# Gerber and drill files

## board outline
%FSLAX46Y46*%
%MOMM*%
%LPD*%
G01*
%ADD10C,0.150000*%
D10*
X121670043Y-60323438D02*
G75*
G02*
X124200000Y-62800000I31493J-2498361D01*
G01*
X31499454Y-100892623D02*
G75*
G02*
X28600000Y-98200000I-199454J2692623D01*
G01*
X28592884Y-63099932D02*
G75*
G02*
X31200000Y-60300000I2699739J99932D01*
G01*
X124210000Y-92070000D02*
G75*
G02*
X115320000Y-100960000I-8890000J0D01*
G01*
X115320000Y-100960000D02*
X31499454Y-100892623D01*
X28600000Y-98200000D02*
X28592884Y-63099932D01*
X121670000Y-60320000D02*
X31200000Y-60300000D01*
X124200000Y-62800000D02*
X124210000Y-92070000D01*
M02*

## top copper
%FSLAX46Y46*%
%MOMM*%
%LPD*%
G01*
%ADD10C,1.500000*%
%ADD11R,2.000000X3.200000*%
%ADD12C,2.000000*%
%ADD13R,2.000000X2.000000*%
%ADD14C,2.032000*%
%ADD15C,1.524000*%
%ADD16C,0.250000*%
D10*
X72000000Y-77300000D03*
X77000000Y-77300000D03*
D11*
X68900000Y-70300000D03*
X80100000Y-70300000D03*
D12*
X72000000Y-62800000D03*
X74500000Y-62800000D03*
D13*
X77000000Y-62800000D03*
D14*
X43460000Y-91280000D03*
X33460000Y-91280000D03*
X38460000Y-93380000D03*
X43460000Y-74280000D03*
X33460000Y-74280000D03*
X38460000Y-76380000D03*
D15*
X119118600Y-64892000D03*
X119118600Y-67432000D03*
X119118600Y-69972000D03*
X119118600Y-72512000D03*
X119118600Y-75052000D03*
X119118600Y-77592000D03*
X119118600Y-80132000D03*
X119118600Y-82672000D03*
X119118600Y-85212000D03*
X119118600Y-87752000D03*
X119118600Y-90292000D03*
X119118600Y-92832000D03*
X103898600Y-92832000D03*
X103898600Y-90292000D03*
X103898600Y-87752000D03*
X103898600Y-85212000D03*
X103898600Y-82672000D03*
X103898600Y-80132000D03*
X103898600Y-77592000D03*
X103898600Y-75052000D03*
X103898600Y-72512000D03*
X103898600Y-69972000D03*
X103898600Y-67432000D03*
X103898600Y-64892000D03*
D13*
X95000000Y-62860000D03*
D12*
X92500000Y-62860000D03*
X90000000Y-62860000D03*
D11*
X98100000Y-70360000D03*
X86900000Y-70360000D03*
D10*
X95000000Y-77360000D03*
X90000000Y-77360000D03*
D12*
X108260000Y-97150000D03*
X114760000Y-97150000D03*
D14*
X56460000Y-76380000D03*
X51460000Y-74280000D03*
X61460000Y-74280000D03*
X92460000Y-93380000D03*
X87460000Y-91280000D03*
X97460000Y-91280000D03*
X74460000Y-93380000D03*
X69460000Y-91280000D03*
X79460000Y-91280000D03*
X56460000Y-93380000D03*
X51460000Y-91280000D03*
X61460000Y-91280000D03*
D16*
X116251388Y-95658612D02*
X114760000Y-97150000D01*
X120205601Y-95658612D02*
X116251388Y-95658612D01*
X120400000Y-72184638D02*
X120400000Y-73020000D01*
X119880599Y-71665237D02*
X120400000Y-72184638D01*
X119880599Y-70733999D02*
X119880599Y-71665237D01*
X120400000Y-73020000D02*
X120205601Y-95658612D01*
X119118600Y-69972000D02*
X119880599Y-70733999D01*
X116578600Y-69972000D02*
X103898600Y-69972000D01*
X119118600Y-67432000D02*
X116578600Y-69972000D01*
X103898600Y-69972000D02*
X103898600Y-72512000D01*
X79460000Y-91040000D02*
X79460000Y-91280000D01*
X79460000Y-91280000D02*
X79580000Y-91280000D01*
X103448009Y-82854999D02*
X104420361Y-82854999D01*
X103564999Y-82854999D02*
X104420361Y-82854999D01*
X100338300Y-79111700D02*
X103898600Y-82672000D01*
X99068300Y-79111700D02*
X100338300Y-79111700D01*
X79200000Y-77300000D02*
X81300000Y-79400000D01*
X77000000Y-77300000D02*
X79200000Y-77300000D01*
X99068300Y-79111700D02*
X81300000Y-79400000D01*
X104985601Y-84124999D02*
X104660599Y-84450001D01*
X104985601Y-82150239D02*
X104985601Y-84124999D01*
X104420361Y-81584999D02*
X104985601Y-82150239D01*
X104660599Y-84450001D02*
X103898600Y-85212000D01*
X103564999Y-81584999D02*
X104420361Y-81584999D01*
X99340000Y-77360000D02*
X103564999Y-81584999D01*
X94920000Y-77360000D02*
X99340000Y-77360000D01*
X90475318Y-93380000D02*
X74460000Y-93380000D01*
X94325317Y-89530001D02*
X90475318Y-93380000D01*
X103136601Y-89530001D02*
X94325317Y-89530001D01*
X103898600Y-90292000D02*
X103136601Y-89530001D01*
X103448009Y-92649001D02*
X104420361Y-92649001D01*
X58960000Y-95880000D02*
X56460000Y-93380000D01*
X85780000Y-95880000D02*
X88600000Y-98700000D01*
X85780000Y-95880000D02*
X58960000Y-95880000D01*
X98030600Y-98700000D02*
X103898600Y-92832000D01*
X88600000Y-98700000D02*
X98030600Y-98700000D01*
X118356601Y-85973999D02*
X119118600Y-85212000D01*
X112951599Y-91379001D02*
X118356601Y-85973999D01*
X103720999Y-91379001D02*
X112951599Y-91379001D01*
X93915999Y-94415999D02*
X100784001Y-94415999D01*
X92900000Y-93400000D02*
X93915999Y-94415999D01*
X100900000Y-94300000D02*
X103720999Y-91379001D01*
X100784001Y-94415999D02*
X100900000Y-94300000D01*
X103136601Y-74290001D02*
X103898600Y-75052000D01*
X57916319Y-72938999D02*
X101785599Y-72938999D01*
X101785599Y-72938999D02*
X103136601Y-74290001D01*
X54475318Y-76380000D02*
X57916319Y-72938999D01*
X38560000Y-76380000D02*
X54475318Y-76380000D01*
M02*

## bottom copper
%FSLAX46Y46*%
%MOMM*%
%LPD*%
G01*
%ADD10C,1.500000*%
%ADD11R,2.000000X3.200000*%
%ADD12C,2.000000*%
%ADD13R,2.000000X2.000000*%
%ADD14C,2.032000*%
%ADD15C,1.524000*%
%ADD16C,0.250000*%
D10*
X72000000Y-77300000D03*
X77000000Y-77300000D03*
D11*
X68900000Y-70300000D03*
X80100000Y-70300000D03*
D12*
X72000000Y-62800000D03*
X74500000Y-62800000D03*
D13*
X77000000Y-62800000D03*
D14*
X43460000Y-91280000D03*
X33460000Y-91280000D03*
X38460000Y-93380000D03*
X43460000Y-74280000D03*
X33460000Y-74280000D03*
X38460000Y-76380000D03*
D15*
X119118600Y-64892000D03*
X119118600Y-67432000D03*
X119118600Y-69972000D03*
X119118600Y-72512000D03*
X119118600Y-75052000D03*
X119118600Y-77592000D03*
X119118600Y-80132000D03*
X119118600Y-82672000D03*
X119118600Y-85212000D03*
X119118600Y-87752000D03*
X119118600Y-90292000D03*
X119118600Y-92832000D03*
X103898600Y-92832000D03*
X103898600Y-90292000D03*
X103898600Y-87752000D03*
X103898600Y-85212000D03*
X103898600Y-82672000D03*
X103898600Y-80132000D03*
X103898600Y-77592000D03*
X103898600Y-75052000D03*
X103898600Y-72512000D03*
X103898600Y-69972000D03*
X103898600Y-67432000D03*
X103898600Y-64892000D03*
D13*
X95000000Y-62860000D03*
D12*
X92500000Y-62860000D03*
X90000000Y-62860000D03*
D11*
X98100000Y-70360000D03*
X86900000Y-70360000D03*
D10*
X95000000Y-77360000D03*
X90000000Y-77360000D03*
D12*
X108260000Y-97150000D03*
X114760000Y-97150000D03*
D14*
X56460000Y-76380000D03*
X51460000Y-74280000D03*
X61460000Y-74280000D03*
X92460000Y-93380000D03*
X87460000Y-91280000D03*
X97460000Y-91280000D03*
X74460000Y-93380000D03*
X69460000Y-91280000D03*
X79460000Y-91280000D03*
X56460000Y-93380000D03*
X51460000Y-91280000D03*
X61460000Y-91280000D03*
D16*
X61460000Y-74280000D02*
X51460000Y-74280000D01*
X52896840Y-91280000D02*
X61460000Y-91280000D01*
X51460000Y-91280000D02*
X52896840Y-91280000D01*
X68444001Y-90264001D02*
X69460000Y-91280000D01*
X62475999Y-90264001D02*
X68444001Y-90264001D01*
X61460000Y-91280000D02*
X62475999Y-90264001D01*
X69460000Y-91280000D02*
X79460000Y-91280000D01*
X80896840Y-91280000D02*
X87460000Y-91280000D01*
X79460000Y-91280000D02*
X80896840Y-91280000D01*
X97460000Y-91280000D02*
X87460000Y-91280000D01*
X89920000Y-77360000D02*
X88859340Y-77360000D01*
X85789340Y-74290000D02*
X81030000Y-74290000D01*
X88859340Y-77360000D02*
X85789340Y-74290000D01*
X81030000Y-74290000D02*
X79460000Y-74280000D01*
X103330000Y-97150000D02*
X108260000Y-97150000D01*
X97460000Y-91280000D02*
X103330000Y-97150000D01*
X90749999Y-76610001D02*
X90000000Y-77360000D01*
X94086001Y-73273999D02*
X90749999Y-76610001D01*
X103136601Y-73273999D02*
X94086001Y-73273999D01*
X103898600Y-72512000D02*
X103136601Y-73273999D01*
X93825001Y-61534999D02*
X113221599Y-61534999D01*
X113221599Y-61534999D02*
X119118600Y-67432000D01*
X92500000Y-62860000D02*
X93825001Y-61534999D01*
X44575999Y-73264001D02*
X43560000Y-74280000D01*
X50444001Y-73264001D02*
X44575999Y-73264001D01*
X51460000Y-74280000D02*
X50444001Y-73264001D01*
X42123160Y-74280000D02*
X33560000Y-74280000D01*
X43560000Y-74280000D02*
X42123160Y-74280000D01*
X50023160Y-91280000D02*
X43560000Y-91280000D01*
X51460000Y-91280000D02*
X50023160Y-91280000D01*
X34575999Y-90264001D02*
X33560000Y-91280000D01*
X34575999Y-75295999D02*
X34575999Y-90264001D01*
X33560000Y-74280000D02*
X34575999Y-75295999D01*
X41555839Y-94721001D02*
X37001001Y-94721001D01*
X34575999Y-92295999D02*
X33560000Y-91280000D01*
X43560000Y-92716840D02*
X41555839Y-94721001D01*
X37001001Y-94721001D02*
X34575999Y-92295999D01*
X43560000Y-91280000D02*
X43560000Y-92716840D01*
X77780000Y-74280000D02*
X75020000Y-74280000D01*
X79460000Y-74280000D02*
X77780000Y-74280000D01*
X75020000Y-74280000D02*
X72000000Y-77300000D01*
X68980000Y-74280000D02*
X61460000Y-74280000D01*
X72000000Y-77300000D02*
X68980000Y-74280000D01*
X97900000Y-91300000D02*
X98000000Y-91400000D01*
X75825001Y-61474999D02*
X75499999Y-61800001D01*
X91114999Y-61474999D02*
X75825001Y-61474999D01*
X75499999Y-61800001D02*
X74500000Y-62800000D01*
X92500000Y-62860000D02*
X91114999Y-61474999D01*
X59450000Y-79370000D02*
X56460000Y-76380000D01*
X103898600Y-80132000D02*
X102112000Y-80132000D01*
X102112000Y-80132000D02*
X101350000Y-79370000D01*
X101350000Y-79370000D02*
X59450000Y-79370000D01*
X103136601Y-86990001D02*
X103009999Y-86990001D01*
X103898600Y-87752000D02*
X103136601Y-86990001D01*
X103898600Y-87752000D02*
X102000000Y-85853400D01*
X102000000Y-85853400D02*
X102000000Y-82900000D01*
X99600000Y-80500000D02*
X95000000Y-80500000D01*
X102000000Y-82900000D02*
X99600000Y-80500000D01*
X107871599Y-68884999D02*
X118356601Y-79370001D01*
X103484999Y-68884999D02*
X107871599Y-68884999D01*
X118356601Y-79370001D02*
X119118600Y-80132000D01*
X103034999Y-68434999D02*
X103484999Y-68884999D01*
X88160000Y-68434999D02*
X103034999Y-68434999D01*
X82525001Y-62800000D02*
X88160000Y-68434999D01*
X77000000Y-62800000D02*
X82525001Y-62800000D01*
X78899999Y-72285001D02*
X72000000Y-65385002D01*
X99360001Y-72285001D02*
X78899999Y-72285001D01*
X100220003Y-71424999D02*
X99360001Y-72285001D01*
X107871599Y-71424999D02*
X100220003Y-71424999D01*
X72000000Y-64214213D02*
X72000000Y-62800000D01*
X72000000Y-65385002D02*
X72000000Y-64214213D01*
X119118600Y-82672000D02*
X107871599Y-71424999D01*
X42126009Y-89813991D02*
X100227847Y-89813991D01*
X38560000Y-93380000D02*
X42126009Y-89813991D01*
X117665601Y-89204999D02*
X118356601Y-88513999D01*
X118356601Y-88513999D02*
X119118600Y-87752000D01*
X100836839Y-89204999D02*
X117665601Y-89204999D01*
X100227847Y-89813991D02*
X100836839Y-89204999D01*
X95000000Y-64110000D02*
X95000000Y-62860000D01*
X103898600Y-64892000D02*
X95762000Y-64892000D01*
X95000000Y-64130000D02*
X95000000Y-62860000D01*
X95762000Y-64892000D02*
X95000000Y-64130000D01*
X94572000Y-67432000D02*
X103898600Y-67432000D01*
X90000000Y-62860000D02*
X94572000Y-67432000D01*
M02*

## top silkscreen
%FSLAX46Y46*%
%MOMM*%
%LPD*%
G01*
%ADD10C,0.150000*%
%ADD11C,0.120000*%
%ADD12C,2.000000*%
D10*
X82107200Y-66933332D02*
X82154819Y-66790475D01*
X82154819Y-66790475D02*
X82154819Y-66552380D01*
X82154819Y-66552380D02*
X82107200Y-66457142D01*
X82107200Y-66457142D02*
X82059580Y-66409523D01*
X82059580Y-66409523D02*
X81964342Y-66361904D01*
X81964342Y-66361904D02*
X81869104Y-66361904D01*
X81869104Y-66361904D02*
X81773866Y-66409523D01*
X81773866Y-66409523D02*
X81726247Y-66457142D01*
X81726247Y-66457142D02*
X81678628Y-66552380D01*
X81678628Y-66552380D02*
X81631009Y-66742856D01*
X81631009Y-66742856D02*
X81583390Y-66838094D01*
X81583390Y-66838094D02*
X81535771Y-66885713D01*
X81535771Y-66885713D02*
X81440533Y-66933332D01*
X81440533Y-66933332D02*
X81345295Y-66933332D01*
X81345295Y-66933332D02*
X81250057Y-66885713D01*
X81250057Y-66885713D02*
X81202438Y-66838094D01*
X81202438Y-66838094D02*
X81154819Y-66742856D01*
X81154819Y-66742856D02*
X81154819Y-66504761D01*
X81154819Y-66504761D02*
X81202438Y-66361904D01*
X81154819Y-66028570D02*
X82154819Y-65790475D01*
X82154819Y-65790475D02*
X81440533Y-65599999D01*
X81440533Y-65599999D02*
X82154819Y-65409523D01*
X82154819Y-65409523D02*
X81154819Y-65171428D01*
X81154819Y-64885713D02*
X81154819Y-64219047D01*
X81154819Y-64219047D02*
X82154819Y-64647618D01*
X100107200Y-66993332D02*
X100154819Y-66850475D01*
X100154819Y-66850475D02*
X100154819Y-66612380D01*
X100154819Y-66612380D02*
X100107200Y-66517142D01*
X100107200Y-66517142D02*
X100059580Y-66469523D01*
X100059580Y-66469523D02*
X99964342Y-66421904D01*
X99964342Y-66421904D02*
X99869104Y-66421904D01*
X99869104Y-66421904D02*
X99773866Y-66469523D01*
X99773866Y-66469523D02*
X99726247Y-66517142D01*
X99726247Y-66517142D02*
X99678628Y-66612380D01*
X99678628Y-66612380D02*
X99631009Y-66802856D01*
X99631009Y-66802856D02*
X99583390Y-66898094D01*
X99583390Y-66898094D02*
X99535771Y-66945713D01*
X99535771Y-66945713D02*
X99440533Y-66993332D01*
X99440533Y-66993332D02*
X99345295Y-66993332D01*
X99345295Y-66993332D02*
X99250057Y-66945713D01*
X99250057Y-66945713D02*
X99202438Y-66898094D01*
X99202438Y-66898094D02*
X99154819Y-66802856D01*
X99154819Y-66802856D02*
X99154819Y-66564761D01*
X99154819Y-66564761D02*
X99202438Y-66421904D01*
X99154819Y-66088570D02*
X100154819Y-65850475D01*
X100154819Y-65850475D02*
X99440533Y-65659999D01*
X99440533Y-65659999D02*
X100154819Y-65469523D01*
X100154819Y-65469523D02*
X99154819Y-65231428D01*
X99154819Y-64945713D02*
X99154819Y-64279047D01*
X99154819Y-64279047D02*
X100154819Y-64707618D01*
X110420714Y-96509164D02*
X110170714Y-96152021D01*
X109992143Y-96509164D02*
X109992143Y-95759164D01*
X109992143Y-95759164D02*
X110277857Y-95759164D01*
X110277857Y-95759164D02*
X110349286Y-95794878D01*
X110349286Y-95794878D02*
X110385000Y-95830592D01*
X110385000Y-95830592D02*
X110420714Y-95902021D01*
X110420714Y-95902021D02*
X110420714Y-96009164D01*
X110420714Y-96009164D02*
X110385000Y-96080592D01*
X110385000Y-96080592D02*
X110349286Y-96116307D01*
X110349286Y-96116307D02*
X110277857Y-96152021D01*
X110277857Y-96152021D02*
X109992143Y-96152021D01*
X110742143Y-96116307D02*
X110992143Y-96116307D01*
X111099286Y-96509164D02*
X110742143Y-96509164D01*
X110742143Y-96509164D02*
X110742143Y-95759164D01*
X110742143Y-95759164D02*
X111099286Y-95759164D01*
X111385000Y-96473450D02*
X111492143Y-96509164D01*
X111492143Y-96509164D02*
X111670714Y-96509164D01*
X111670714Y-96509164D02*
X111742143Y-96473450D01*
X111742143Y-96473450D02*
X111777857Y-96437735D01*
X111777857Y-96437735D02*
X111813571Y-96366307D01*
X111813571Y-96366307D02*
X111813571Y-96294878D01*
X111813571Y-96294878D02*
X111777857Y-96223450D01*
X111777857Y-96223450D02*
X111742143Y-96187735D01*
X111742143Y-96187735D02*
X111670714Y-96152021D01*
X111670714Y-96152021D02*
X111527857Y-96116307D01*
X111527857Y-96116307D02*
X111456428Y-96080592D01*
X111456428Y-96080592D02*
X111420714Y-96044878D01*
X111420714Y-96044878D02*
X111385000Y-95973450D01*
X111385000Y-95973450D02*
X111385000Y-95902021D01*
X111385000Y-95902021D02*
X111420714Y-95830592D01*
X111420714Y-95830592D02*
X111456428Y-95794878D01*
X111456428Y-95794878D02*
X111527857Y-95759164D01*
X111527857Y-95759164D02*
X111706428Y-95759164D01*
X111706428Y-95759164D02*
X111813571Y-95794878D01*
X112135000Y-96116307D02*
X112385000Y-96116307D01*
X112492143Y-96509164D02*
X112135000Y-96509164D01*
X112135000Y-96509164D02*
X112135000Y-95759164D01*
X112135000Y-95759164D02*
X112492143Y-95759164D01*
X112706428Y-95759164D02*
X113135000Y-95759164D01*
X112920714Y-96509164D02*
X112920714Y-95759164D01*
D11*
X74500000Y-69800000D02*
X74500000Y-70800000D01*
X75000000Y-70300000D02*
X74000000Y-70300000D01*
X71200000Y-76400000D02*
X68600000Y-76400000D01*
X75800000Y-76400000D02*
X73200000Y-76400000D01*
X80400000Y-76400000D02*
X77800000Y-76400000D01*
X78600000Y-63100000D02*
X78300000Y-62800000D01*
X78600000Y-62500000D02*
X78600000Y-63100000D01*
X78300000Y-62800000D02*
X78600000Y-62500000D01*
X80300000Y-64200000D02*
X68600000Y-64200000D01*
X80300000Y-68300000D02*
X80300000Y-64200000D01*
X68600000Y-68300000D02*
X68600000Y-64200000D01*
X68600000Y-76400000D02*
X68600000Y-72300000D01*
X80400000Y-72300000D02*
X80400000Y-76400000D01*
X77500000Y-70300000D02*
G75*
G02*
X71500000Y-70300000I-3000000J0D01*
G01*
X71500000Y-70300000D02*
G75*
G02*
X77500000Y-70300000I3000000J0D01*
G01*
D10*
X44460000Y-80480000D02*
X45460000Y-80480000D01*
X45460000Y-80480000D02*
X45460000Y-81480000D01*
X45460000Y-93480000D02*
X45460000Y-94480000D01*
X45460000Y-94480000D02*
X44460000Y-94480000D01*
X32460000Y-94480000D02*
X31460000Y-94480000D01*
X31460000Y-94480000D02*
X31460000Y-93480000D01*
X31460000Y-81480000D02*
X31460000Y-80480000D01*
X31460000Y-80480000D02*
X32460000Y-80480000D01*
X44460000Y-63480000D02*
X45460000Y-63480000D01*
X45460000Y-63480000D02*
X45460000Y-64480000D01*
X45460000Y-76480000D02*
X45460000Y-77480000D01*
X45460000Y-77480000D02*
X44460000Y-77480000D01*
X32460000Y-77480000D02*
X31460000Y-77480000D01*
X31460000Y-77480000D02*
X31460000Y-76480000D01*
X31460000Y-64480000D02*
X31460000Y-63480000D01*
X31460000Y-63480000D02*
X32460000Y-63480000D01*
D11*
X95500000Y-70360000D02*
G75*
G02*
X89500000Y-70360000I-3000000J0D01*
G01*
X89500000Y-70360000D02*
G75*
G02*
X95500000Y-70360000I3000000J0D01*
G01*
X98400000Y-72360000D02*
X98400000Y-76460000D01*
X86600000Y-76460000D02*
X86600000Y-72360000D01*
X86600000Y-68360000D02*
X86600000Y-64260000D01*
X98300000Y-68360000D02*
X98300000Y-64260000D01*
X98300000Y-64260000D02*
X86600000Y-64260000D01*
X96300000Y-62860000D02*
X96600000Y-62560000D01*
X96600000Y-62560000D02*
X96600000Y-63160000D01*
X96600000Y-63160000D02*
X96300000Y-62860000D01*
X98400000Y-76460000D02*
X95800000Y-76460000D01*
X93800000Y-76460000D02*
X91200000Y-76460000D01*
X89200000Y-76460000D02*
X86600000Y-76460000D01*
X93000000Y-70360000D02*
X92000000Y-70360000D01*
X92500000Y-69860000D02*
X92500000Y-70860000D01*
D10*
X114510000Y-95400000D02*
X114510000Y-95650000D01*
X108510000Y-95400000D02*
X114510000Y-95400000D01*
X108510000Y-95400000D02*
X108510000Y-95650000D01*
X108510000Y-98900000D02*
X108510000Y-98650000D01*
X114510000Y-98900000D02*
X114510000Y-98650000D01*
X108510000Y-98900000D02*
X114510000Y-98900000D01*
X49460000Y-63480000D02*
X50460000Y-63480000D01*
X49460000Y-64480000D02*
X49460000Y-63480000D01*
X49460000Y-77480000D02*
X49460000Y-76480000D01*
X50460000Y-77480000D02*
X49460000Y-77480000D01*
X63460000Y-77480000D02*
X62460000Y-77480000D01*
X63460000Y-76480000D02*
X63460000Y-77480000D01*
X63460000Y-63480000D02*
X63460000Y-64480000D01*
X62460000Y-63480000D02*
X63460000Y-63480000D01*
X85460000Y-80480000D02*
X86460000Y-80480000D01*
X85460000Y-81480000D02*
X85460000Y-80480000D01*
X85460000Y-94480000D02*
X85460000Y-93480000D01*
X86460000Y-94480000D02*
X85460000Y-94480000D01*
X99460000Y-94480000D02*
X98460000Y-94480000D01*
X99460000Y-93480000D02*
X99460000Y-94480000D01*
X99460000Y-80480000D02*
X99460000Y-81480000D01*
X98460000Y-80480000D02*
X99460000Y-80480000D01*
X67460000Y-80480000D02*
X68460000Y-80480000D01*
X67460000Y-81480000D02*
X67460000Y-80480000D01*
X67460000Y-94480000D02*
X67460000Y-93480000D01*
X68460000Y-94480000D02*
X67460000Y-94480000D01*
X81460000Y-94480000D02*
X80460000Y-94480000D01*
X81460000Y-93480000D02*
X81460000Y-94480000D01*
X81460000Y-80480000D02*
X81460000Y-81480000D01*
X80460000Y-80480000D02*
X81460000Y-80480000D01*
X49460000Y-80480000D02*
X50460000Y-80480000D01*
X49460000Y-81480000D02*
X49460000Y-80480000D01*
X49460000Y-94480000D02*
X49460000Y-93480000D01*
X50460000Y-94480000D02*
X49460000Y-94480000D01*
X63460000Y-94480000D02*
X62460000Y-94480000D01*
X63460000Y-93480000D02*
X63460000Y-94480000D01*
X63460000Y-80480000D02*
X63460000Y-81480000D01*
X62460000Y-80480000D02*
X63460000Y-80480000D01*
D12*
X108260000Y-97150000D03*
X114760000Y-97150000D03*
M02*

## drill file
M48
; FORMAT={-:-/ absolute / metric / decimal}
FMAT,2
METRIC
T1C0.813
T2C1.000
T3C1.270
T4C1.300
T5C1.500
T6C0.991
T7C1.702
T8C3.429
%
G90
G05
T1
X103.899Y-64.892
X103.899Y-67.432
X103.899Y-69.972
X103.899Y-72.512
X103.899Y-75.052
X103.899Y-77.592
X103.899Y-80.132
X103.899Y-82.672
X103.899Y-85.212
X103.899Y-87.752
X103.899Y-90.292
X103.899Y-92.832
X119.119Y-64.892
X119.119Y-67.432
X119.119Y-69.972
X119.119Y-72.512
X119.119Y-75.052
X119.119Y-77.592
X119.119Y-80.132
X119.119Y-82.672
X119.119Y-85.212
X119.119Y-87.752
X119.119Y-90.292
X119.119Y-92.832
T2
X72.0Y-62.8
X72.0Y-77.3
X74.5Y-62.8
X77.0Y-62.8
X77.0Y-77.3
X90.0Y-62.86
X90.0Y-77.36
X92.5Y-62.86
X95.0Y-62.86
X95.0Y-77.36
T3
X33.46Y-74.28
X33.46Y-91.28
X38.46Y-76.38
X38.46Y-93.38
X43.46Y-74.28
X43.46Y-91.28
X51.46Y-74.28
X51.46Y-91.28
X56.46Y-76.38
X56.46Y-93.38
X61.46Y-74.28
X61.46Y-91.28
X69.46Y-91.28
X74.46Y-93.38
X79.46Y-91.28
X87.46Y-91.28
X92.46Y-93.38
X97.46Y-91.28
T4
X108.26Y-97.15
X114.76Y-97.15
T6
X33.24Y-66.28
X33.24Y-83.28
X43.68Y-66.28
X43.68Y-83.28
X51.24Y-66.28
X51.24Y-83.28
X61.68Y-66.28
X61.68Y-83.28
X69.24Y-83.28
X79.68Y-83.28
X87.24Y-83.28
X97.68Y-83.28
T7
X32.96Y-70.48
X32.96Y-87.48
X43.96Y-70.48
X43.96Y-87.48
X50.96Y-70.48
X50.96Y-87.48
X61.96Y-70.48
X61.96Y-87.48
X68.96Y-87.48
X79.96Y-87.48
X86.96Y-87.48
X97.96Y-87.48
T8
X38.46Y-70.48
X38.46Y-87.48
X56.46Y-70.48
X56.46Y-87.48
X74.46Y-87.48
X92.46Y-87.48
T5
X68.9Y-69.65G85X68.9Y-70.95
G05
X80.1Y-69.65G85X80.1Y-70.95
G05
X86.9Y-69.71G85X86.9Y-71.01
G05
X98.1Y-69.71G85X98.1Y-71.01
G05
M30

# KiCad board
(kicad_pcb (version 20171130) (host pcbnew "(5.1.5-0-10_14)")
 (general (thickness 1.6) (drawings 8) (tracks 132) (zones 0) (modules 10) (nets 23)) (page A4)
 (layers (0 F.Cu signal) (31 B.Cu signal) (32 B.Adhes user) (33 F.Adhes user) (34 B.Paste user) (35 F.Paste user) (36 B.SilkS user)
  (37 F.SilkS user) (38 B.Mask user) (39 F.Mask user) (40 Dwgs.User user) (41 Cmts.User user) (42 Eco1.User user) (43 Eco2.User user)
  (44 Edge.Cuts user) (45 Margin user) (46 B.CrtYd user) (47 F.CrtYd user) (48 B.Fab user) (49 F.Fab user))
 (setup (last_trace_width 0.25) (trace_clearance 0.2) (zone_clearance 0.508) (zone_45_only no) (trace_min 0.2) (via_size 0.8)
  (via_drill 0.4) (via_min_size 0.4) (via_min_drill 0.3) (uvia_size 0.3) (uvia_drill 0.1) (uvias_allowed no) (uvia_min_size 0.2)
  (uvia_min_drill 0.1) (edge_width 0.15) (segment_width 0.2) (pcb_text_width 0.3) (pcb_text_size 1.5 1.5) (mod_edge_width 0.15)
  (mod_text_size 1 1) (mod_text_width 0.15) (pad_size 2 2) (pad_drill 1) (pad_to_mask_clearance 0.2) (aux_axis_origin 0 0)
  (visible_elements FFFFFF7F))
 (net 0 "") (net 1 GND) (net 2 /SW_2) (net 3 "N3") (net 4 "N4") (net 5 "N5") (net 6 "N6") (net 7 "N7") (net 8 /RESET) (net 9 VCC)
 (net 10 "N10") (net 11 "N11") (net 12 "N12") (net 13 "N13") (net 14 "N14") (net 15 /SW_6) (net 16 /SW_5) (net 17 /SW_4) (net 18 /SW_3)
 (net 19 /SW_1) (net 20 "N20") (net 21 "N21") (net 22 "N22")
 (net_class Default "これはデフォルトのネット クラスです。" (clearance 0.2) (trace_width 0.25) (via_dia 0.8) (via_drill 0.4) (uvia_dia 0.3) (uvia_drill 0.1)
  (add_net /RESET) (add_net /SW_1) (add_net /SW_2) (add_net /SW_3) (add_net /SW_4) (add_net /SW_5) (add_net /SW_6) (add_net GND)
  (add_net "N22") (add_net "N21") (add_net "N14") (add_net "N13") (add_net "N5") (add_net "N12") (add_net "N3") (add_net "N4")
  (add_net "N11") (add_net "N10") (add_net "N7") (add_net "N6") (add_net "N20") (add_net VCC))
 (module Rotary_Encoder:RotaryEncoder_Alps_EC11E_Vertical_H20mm (layer F.Cu) (at 77 62.8 270)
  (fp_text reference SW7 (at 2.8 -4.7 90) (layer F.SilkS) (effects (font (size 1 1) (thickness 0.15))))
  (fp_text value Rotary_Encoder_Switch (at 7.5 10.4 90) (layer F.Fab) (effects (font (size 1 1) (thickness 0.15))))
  (fp_line (start 7 2.5) (end 8 2.5) (layer F.SilkS) (width 0.12))
  (fp_line (start 7.5 2) (end 7.5 3) (layer F.SilkS) (width 0.12))
  (fp_line (start 13.6 5.8) (end 13.6 8.4) (layer F.SilkS) (width 0.12))
  (fp_line (start 13.6 1.2) (end 13.6 3.8) (layer F.SilkS) (width 0.12))
  (fp_line (start 13.6 -3.4) (end 13.6 -0.8) (layer F.SilkS) (width 0.12))
  (fp_line (start 0.3 -1.6) (end 0 -1.3) (layer F.SilkS) (width 0.12))
  (fp_line (start -0.3 -1.6) (end 0.3 -1.6) (layer F.SilkS) (width 0.12))
  (fp_line (start 0 -1.3) (end -0.3 -1.6) (layer F.SilkS) (width 0.12))
  (fp_line (start 1.4 -3.3) (end 1.4 8.4) (layer F.SilkS) (width 0.12))
  (fp_line (start 5.5 -3.3) (end 1.4 -3.3) (layer F.SilkS) (width 0.12))
  (fp_line (start 5.5 8.4) (end 1.4 8.4) (layer F.SilkS) (width 0.12))
  (fp_line (start 13.6 8.4) (end 9.5 8.4) (layer F.SilkS) (width 0.12))
  (fp_line (start 9.5 -3.4) (end 13.6 -3.4) (layer F.SilkS) (width 0.12))
  (fp_circle (center 7.5 2.5) (end 10.5 2.5) (layer F.SilkS) (width 0.12))
  (pad "" thru_hole circle (at 14.5 5 270) (size 1.5 1.5) (drill 1) (layers *.Cu *.Mask) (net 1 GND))
  (pad "" thru_hole circle (at 14.5 0 270) (size 1.5 1.5) (drill 1) (layers *.Cu *.Mask) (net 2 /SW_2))
  (pad MP thru_hole rect (at 7.5 8.1 270) (size 3.2 2) (drill oval 2.8 1.5) (layers *.Cu *.Mask))
  (pad MP thru_hole rect (at 7.5 -3.1 270) (size 3.2 2) (drill oval 2.8 1.5) (layers *.Cu *.Mask))
  (pad B thru_hole circle (at 0 5 270) (size 2 2) (drill 1) (layers *.Cu *.Mask) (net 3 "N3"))
  (pad C thru_hole circle (at 0 2.5 270) (size 2 2) (drill 1) (layers *.Cu *.Mask) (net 1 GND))
  (pad A thru_hole rect (at 0 0 270) (size 2 2) (drill 1) (layers *.Cu *.Mask) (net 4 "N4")))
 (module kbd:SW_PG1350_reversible (layer F.Cu) (at 38.46 87.48)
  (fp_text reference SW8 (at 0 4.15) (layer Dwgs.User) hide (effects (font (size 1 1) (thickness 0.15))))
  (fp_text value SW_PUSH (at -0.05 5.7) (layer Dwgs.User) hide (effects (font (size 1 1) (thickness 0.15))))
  (fp_line (start 6 -7) (end 7 -7) (layer F.SilkS) (width 0.15))
  (fp_line (start 7 -7) (end 7 -6) (layer F.SilkS) (width 0.15)) (fp_line (start 7 6) (end 7 7) (layer F.SilkS) (width 0.15))
  (fp_line (start 7 7) (end 6 7) (layer F.SilkS) (width 0.15))
  (fp_line (start -6 7) (end -7 7) (layer F.SilkS) (width 0.15))
  (fp_line (start -7 7) (end -7 6) (layer F.SilkS) (width 0.15))
  (fp_line (start -7 -6) (end -7 -7) (layer F.SilkS) (width 0.15))
  (fp_line (start -7 -7) (end -6 -7) (layer F.SilkS) (width 0.15))
  (pad "" np_thru_hole circle (at -5.22 -4.2) (size 0.9906 0.9906) (drill 0.9906) (layers *.Cu *.Mask))
  (pad 2 thru_hole circle (at 5 3.8) (size 2.032 2.032) (drill 1.27) (layers *.Cu *.Mask) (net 1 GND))
  (pad "" np_thru_hole circle (at 0 0) (size 3.429 3.429) (drill 3.429) (layers *.Cu *.Mask))
  (pad 2 thru_hole circle (at -5 3.8) (size 2.032 2.032) (drill 1.27) (layers *.Cu *.Mask) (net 1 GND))
  (pad 1 thru_hole circle (at 0 5.9) (size 2.032 2.032) (drill 1.27) (layers *.Cu *.Mask) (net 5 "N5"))
  (pad "" np_thru_hole circle (at 5.22 -4.2) (size 0.9906 0.9906) (drill 0.9906) (layers *.Cu *.Mask))
  (pad "" np_thru_hole circle (at 5.5 0) (size 1.7018 1.7018) (drill 1.7018) (layers *.Cu *.Mask))
  (pad "" np_thru_hole circle (at -5.5 0) (size 1.7018 1.7018) (drill 1.7018) (layers *.Cu *.Mask)))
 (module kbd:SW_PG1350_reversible (layer F.Cu) (at 38.46 70.48)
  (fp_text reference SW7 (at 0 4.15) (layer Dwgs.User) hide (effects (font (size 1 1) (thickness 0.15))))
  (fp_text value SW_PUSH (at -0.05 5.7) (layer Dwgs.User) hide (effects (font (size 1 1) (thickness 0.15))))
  (fp_line (start 6 -7) (end 7 -7) (layer F.SilkS) (width 0.15))
  (fp_line (start 7 -7) (end 7 -6) (layer F.SilkS) (width 0.15)) (fp_line (start 7 6) (end 7 7) (layer F.SilkS) (width 0.15))
  (fp_line (start 7 7) (end 6 7) (layer F.SilkS) (width 0.15))
  (fp_line (start -6 7) (end -7 7) (layer F.SilkS) (width 0.15))
  (fp_line (start -7 7) (end -7 6) (layer F.SilkS) (width 0.15))
  (fp_line (start -7 -6) (end -7 -7) (layer F.SilkS) (width 0.15))
  (fp_line (start -7 -7) (end -6 -7) (layer F.SilkS) (width 0.15))
  (pad "" np_thru_hole circle (at -5.22 -4.2) (size 0.9906 0.9906) (drill 0.9906) (layers *.Cu *.Mask))
  (pad 2 thru_hole circle (at 5 3.8) (size 2.032 2.032) (drill 1.27) (layers *.Cu *.Mask) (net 1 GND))
  (pad "" np_thru_hole circle (at 0 0) (size 3.429 3.429) (drill 3.429) (layers *.Cu *.Mask))
  (pad 2 thru_hole circle (at -5 3.8) (size 2.032 2.032) (drill 1.27) (layers *.Cu *.Mask) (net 1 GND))
  (pad 1 thru_hole circle (at 0 5.9) (size 2.032 2.032) (drill 1.27) (layers *.Cu *.Mask) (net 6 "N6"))
  (pad "" np_thru_hole circle (at 5.22 -4.2) (size 0.9906 0.9906) (drill 0.9906) (layers *.Cu *.Mask))
  (pad "" np_thru_hole circle (at 5.5 0) (size 1.7018 1.7018) (drill 1.7018) (layers *.Cu *.Mask))
  (pad "" np_thru_hole circle (at -5.5 0) (size 1.7018 1.7018) (drill 1.7018) (layers *.Cu *.Mask)))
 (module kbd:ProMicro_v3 (layer B.Cu) (at 111.51 79.37 180)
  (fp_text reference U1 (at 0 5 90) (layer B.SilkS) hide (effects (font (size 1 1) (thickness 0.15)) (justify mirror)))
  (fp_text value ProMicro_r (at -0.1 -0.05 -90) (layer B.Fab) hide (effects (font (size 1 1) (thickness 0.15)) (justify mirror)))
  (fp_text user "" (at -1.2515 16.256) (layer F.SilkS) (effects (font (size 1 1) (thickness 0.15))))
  (pad 24 thru_hole circle (at -7.6086 14.478 180) (size 1.524 1.524) (drill 0.8128) (layers *.Cu *.Mask B.SilkS) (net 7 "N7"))
  (pad 23 thru_hole circle (at -7.6086 11.938 180) (size 1.524 1.524) (drill 0.8128) (layers *.Cu *.Mask B.SilkS) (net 1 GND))
  (pad 22 thru_hole circle (at -7.6086 9.398 180) (size 1.524 1.524) (drill 0.8128) (layers *.Cu *.Mask B.SilkS) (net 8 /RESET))
  (pad 21 thru_hole circle (at -7.6086 6.858 180) (size 1.524 1.524) (drill 0.8128) (layers *.Cu *.Mask B.SilkS) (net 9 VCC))
  (pad 20 thru_hole circle (at -7.6086 4.318 180) (size 1.524 1.524) (drill 0.8128) (layers *.Cu *.Mask B.SilkS) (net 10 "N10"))
  (pad 19 thru_hole circle (at -7.6086 1.778 180) (size 1.524 1.524) (drill 0.8128) (layers *.Cu *.Mask B.SilkS) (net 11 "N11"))
  (pad 18 thru_hole circle (at -7.6086 -0.762 180) (size 1.524 1.524) (drill 0.8128) (layers *.Cu *.Mask B.SilkS) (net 4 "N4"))
  (pad 17 thru_hole circle (at -7.6086 -3.302 180) (size 1.524 1.524) (drill 0.8128) (layers *.Cu *.Mask B.SilkS) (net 3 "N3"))
  (pad 16 thru_hole circle (at -7.6086 -5.842 180) (size 1.524 1.524) (drill 0.8128) (layers *.Cu *.Mask B.SilkS) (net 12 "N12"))
  (pad 15 thru_hole circle (at -7.6086 -8.382 180) (size 1.524 1.524) (drill 0.8128) (layers *.Cu *.Mask B.SilkS) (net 5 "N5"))
  (pad 14 thru_hole circle (at -7.6086 -10.922 180) (size 1.524 1.524) (drill 0.8128) (layers *.Cu *.Mask B.SilkS) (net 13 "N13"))
  (pad 13 thru_hole circle (at -7.6086 -13.462 180) (size 1.524 1.524) (drill 0.8128) (layers *.Cu *.Mask B.SilkS) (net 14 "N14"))
  (pad 12 thru_hole circle (at 7.6114 -13.462 180) (size 1.524 1.524) (drill 0.8128) (layers *.Cu *.Mask B.SilkS) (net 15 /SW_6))
  (pad 11 thru_hole circle (at 7.6114 -10.922 180) (size 1.524 1.524) (drill 0.8128) (layers *.Cu *.Mask B.SilkS) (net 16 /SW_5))
  (pad 10 thru_hole circle (at 7.6114 -8.382 180) (size 1.524 1.524) (drill 0.8128) (layers *.Cu *.Mask B.SilkS) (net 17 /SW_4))
  (pad 9 thru_hole circle (at 7.6114 -5.842 180) (size 1.524 1.524) (drill 0.8128) (layers *.Cu *.Mask B.SilkS) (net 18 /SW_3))
  (pad 8 thru_hole circle (at 7.6114 -3.302 180) (size 1.524 1.524) (drill 0.8128) (layers *.Cu *.Mask B.SilkS) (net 2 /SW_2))
  (pad 7 thru_hole circle (at 7.6114 -0.762 180) (size 1.524 1.524) (drill 0.8128) (layers *.Cu *.Mask B.SilkS) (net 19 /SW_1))
  (pad 6 thru_hole circle (at 7.6114 1.778 180) (size 1.524 1.524) (drill 0.8128) (layers *.Cu *.Mask B.SilkS) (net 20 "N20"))
  (pad 5 thru_hole circle (at 7.6114 4.318 180) (size 1.524 1.524) (drill 0.8128) (layers *.Cu *.Mask B.SilkS) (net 6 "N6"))
  (pad 4 thru_hole circle (at 7.6114 6.858 180) (size 1.524 1.524) (drill 0.8128) (layers *.Cu *.Mask B.SilkS) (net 1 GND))
  (pad 3 thru_hole circle (at 7.6114 9.398 180) (size 1.524 1.524) (drill 0.8128) (layers *.Cu *.Mask B.SilkS) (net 1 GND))
  (pad 2 thru_hole circle (at 7.6114 11.938 180) (size 1.524 1.524) (drill 0.8128) (layers *.Cu *.Mask B.SilkS) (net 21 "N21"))
  (pad 1 thru_hole circle (at 7.6114 14.478 180) (size 1.524 1.524) (drill 0.8128) (layers *.Cu *.Mask B.SilkS) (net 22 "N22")))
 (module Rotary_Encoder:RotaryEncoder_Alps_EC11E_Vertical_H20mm (layer F.Cu) (at 95 62.86 270)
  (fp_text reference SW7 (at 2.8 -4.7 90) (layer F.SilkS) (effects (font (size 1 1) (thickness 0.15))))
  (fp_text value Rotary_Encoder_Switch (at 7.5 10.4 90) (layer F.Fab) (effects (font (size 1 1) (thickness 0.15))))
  (fp_circle (center 7.5 2.5) (end 10.5 2.5) (layer F.SilkS) (width 0.12))
  (fp_line (start 9.5 -3.4) (end 13.6 -3.4) (layer F.SilkS) (width 0.12))
  (fp_line (start 13.6 8.4) (end 9.5 8.4) (layer F.SilkS) (width 0.12))
  (fp_line (start 5.5 8.4) (end 1.4 8.4) (layer F.SilkS) (width 0.12))
  (fp_line (start 5.5 -3.3) (end 1.4 -3.3) (layer F.SilkS) (width 0.12))
  (fp_line (start 1.4 -3.3) (end 1.4 8.4) (layer F.SilkS) (width 0.12))
  (fp_line (start 0 -1.3) (end -0.3 -1.6) (layer F.SilkS) (width 0.12))
  (fp_line (start -0.3 -1.6) (end 0.3 -1.6) (layer F.SilkS) (width 0.12))
  (fp_line (start 0.3 -1.6) (end 0 -1.3) (layer F.SilkS) (width 0.12))
  (fp_line (start 13.6 -3.4) (end 13.6 -0.8) (layer F.SilkS) (width 0.12))
  (fp_line (start 13.6 1.2) (end 13.6 3.8) (layer F.SilkS) (width 0.12))
  (fp_line (start 13.6 5.8) (end 13.6 8.4) (layer F.SilkS) (width 0.12))
  (fp_line (start 7.5 2) (end 7.5 3) (layer F.SilkS) (width 0.12))
  (fp_line (start 7 2.5) (end 8 2.5) (layer F.SilkS) (width 0.12))
  (pad A thru_hole rect (at 0 0 270) (size 2 2) (drill 1) (layers *.Cu *.Mask) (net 22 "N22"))
  (pad C thru_hole circle (at 0 2.5 270) (size 2 2) (drill 1) (layers *.Cu *.Mask) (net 1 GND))
  (pad B thru_hole circle (at 0 5 270) (size 2 2) (drill 1) (layers *.Cu *.Mask) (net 21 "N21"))
  (pad MP thru_hole rect (at 7.5 -3.1 270) (size 3.2 2) (drill oval 2.8 1.5) (layers *.Cu *.Mask))
  (pad MP thru_hole rect (at 7.5 8.1 270) (size 3.2 2) (drill oval 2.8 1.5) (layers *.Cu *.Mask))
  (pad "" thru_hole circle (at 14.5 0 270) (size 1.5 1.5) (drill 1) (layers *.Cu *.Mask) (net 18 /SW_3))
  (pad "" thru_hole circle (at 14.5 5 270) (size 1.5 1.5) (drill 1) (layers *.Cu *.Mask) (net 1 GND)))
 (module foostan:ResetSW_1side (layer F.Cu) (at 111.51 97.15)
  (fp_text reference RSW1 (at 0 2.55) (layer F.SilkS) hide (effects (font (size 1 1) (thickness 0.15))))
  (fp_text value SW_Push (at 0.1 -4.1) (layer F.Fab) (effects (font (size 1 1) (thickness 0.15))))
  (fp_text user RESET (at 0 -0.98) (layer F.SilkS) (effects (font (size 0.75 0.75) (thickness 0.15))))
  (fp_line (start 3 -1.75) (end 3 -1.5) (layer F.SilkS) (width 0.15))
  (fp_line (start -3 -1.75) (end 3 -1.75) (layer F.SilkS) (width 0.15))
  (fp_line (start -3 -1.75) (end -3 -1.5) (layer F.SilkS) (width 0.15))
  (fp_line (start -3 1.75) (end -3 1.5) (layer F.SilkS) (width 0.15))
  (fp_line (start 3 1.75) (end 3 1.5) (layer F.SilkS) (width 0.15))
  (fp_line (start -3 1.75) (end 3 1.75) (layer F.SilkS) (width 0.15))
  (pad 2 thru_hole circle (at -3.25 0) (size 2 2) (drill 1.3) (layers *.Cu F.SilkS B.Mask) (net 1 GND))
  (pad 1 thru_hole circle (at 3.25 0) (size 2 2) (drill 1.3) (layers *.Cu F.SilkS B.Mask) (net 8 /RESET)))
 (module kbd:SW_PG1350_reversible (layer F.Cu) (at 56.46 70.48)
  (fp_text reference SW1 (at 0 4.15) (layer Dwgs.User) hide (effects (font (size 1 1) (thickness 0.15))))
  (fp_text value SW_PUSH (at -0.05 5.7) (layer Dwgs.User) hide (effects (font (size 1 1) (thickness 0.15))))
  (fp_line (start -7 -7) (end -6 -7) (layer F.SilkS) (width 0.15))
  (fp_line (start -7 -6) (end -7 -7) (layer F.SilkS) (width 0.15))
  (fp_line (start -7 7) (end -7 6) (layer F.SilkS) (width 0.15))
  (fp_line (start -6 7) (end -7 7) (layer F.SilkS) (width 0.15)) (fp_line (start 7 7) (end 6 7) (layer F.SilkS) (width 0.15))
  (fp_line (start 7 6) (end 7 7) (layer F.SilkS) (width 0.15))
  (fp_line (start 7 -7) (end 7 -6) (layer F.SilkS) (width 0.15))
  (fp_line (start 6 -7) (end 7 -7) (layer F.SilkS) (width 0.15))
  (pad "" np_thru_hole circle (at -5.5 0) (size 1.7018 1.7018) (drill 1.7018) (layers *.Cu *.Mask))
  (pad "" np_thru_hole circle (at 5.5 0) (size 1.7018 1.7018) (drill 1.7018) (layers *.Cu *.Mask))
  (pad "" np_thru_hole circle (at 5.22 -4.2) (size 0.9906 0.9906) (drill 0.9906) (layers *.Cu *.Mask))
  (pad 1 thru_hole circle (at 0 5.9) (size 2.032 2.032) (drill 1.27) (layers *.Cu *.Mask) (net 19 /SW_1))
  (pad 2 thru_hole circle (at -5 3.8) (size 2.032 2.032) (drill 1.27) (layers *.Cu *.Mask) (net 1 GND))
  (pad "" np_thru_hole circle (at 0 0) (size 3.429 3.429) (drill 3.429) (layers *.Cu *.Mask))
  (pad 2 thru_hole circle (at 5 3.8) (size 2.032 2.032) (drill 1.27) (layers *.Cu *.Mask) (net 1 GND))
  (pad "" np_thru_hole circle (at -5.22 -4.2) (size 0.9906 0.9906) (drill 0.9906) (layers *.Cu *.Mask)))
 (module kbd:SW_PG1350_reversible (layer F.Cu) (at 92.46 87.48)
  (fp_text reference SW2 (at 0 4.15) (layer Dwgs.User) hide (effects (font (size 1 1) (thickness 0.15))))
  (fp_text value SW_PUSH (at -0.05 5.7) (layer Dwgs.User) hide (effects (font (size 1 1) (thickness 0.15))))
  (fp_line (start -7 -7) (end -6 -7) (layer F.SilkS) (width 0.15))
  (fp_line (start -7 -6) (end -7 -7) (layer F.SilkS) (width 0.15))
  (fp_line (start -7 7) (end -7 6) (layer F.SilkS) (width 0.15))
  (fp_line (start -6 7) (end -7 7) (layer F.SilkS) (width 0.15)) (fp_line (start 7 7) (end 6 7) (layer F.SilkS) (width 0.15))
  (fp_line (start 7 6) (end 7 7) (layer F.SilkS) (width 0.15))
  (fp_line (start 7 -7) (end 7 -6) (layer F.SilkS) (width 0.15))
  (fp_line (start 6 -7) (end 7 -7) (layer F.SilkS) (width 0.15))
  (pad "" np_thru_hole circle (at -5.5 0) (size 1.7018 1.7018) (drill 1.7018) (layers *.Cu *.Mask))
  (pad "" np_thru_hole circle (at 5.5 0) (size 1.7018 1.7018) (drill 1.7018) (layers *.Cu *.Mask))
  (pad "" np_thru_hole circle (at 5.22 -4.2) (size 0.9906 0.9906) (drill 0.9906) (layers *.Cu *.Mask))
  (pad 1 thru_hole circle (at 0 5.9) (size 2.032 2.032) (drill 1.27) (layers *.Cu *.Mask) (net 12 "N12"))
  (pad 2 thru_hole circle (at -5 3.8) (size 2.032 2.032) (drill 1.27) (layers *.Cu *.Mask) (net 1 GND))
  (pad "" np_thru_hole circle (at 0 0) (size 3.429 3.429) (drill 3.429) (layers *.Cu *.Mask))
  (pad 2 thru_hole circle (at 5 3.8) (size 2.032 2.032) (drill 1.27) (layers *.Cu *.Mask) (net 1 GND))
  (pad "" np_thru_hole circle (at -5.22 -4.2) (size 0.9906 0.9906) (drill 0.9906) (layers *.Cu *.Mask)))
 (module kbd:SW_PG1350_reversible (layer F.Cu) (at 74.46 87.48)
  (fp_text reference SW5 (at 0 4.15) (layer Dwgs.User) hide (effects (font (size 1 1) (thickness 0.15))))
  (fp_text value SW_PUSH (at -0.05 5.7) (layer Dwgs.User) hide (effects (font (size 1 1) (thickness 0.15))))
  (fp_line (start -7 -7) (end -6 -7) (layer F.SilkS) (width 0.15))
  (fp_line (start -7 -6) (end -7 -7) (layer F.SilkS) (width 0.15))
  (fp_line (start -7 7) (end -7 6) (layer F.SilkS) (width 0.15))
  (fp_line (start -6 7) (end -7 7) (layer F.SilkS) (width 0.15)) (fp_line (start 7 7) (end 6 7) (layer F.SilkS) (width 0.15))
  (fp_line (start 7 6) (end 7 7) (layer F.SilkS) (width 0.15))
  (fp_line (start 7 -7) (end 7 -6) (layer F.SilkS) (width 0.15))
  (fp_line (start 6 -7) (end 7 -7) (layer F.SilkS) (width 0.15))
  (pad "" np_thru_hole circle (at -5.5 0) (size 1.7018 1.7018) (drill 1.7018) (layers *.Cu *.Mask))
  (pad "" np_thru_hole circle (at 5.5 0) (size 1.7018 1.7018) (drill 1.7018) (layers *.Cu *.Mask))
  (pad "" np_thru_hole circle (at 5.22 -4.2) (size 0.9906 0.9906) (drill 0.9906) (layers *.Cu *.Mask))
  (pad 1 thru_hole circle (at 0 5.9) (size 2.032 2.032) (drill 1.27) (layers *.Cu *.Mask) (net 16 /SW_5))
  (pad 2 thru_hole circle (at -5 3.8) (size 2.032 2.032) (drill 1.27) (layers *.Cu *.Mask) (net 1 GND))
  (pad "" np_thru_hole circle (at 0 0) (size 3.429 3.429) (drill 3.429) (layers *.Cu *.Mask))
  (pad 2 thru_hole circle (at 5 3.8) (size 2.032 2.032) (drill 1.27) (layers *.Cu *.Mask) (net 1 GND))
  (pad "" np_thru_hole circle (at -5.22 -4.2) (size 0.9906 0.9906) (drill 0.9906) (layers *.Cu *.Mask)))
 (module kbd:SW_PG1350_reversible (layer F.Cu) (at 56.46 87.48)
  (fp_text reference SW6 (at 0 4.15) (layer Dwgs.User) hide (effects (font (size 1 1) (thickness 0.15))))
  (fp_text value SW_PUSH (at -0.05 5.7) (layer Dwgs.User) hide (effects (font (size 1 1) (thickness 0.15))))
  (fp_line (start -7 -7) (end -6 -7) (layer F.SilkS) (width 0.15))
  (fp_line (start -7 -6) (end -7 -7) (layer F.SilkS) (width 0.15))
  (fp_line (start -7 7) (end -7 6) (layer F.SilkS) (width 0.15))
  (fp_line (start -6 7) (end -7 7) (layer F.SilkS) (width 0.15)) (fp_line (start 7 7) (end 6 7) (layer F.SilkS) (width 0.15))
  (fp_line (start 7 6) (end 7 7) (layer F.SilkS) (width 0.15))
  (fp_line (start 7 -7) (end 7 -6) (layer F.SilkS) (width 0.15))
  (fp_line (start 6 -7) (end 7 -7) (layer F.SilkS) (width 0.15))
  (pad "" np_thru_hole circle (at -5.5 0) (size 1.7018 1.7018) (drill 1.7018) (layers *.Cu *.Mask))
  (pad "" np_thru_hole circle (at 5.5 0) (size 1.7018 1.7018) (drill 1.7018) (layers *.Cu *.Mask))
  (pad "" np_thru_hole circle (at 5.22 -4.2) (size 0.9906 0.9906) (drill 0.9906) (layers *.Cu *.Mask))
  (pad 1 thru_hole circle (at 0 5.9) (size 2.032 2.032) (drill 1.27) (layers *.Cu *.Mask) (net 15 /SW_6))
  (pad 2 thru_hole circle (at -5 3.8) (size 2.032 2.032) (drill 1.27) (layers *.Cu *.Mask) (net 1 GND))
  (pad "" np_thru_hole circle (at 0 0) (size 3.429 3.429) (drill 3.429) (layers *.Cu *.Mask))
  (pad 2 thru_hole circle (at 5 3.8) (size 2.032 2.032) (drill 1.27) (layers *.Cu *.Mask) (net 1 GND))
  (pad "" np_thru_hole circle (at -5.22 -4.2) (size 0.9906 0.9906) (drill 0.9906) (layers *.Cu *.Mask)))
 (gr_arc (start 121.701536 62.821799) (end 124.2 62.8) (angle -90.22231091) (layer Edge.Cuts) (width 0.15))
 (gr_arc (start 31.3 98.2) (end 28.6 98.2) (angle -94.2363948) (layer Edge.Cuts) (width 0.15))
 (gr_arc (start 31.292623 63) (end 31.2 60.3) (angle -90.15510012) (layer Edge.Cuts) (width 0.15))
 (gr_arc (start 115.32 92.07) (end 115.32 100.96) (angle -90) (layer Edge.Cuts) (width 0.15))
 (gr_line (start 115.32 100.96) (end 31.499454 100.892623) (layer Edge.Cuts) (width 0.15))
 (gr_line (start 28.6 98.2) (end 28.592884 63.099932) (layer Edge.Cuts) (width 0.15))
 (gr_line (start 121.67 60.32) (end 31.2 60.3) (layer Edge.Cuts) (width 0.15))
 (gr_line (start 124.2 62.8) (end 124.21 92.07) (layer Edge.Cuts) (width 0.15))
 (segment (start 116.251388 95.658612) (end 114.76 97.15) (width 0.25) (layer F.Cu) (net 8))
 (segment (start 120.205601 95.658612) (end 116.251388 95.658612) (width 0.25) (layer F.Cu) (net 8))
 (segment (start 120.4 72.184638) (end 120.4 73.02) (width 0.25) (layer F.Cu) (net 8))
 (segment (start 119.880599 71.665237) (end 120.4 72.184638) (width 0.25) (layer F.Cu) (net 8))
 (segment (start 119.880599 70.733999) (end 119.880599 71.665237) (width 0.25) (layer F.Cu) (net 8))
 (segment (start 120.4 73.02) (end 120.205601 95.658612) (width 0.25) (layer F.Cu) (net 8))
 (segment (start 119.1186 69.972) (end 119.880599 70.733999) (width 0.25) (layer F.Cu) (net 8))
 (segment (start 61.46 74.28) (end 51.46 74.28) (width 0.25) (layer B.Cu) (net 1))
 (segment (start 52.89684 91.28) (end 61.46 91.28) (width 0.25) (layer B.Cu) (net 1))
 (segment (start 51.46 91.28) (end 52.89684 91.28) (width 0.25) (layer B.Cu) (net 1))
 (segment (start 68.444001 90.264001) (end 69.46 91.28) (width 0.25) (layer B.Cu) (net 1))
 (segment (start 62.475999 90.264001) (end 68.444001 90.264001) (width 0.25) (layer B.Cu) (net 1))
 (segment (start 61.46 91.28) (end 62.475999 90.264001) (width 0.25) (layer B.Cu) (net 1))
 (segment (start 69.46 91.28) (end 79.46 91.28) (width 0.25) (layer B.Cu) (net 1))
 (segment (start 80.89684 91.28) (end 87.46 91.28) (width 0.25) (layer B.Cu) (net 1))
 (segment (start 79.46 91.28) (end 80.89684 91.28) (width 0.25) (layer B.Cu) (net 1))
 (segment (start 97.46 91.28) (end 87.46 91.28) (width 0.25) (layer B.Cu) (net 1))
 (segment (start 89.92 77.36) (end 88.85934 77.36) (width 0.25) (layer B.Cu) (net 1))
 (segment (start 85.78934 74.29) (end 81.03 74.29) (width 0.25) (layer B.Cu) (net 1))
 (segment (start 88.85934 77.36) (end 85.78934 74.29) (width 0.25) (layer B.Cu) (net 1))
 (segment (start 81.03 74.29) (end 79.46 74.28) (width 0.25) (layer B.Cu) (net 1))
 (segment (start 103.33 97.15) (end 108.26 97.15) (width 0.25) (layer B.Cu) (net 1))
 (segment (start 97.46 91.28) (end 103.33 97.15) (width 0.25) (layer B.Cu) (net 1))
 (segment (start 90.749999 76.610001) (end 90 77.36) (width 0.25) (layer B.Cu) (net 1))
 (segment (start 94.086001 73.273999) (end 90.749999 76.610001) (width 0.25) (layer B.Cu) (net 1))
 (segment (start 103.136601 73.273999) (end 94.086001 73.273999) (width 0.25) (layer B.Cu) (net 1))
 (segment (start 103.8986 72.512) (end 103.136601 73.273999) (width 0.25) (layer B.Cu) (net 1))
 (segment (start 116.5786 69.972) (end 103.8986 69.972) (width 0.25) (layer F.Cu) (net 1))
 (segment (start 119.1186 67.432) (end 116.5786 69.972) (width 0.25) (layer F.Cu) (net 1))
 (segment (start 103.8986 69.972) (end 103.8986 72.512) (width 0.25) (layer F.Cu) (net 1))
 (segment (start 93.825001 61.534999) (end 113.221599 61.534999) (width 0.25) (layer B.Cu) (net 1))
 (segment (start 113.221599 61.534999) (end 119.1186 67.432) (width 0.25) (layer B.Cu) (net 1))
 (segment (start 92.5 62.86) (end 93.825001 61.534999) (width 0.25) (layer B.Cu) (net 1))
 (segment (start 44.575999 73.264001) (end 43.56 74.28) (width 0.25) (layer B.Cu) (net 1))
 (segment (start 50.444001 73.264001) (end 44.575999 73.264001) (width 0.25) (layer B.Cu) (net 1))
 (segment (start 51.46 74.28) (end 50.444001 73.264001) (width 0.25) (layer B.Cu) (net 1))
 (segment (start 42.12316 74.28) (end 33.56 74.28) (width 0.25) (layer B.Cu) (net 1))
 (segment (start 43.56 74.28) (end 42.12316 74.28) (width 0.25) (layer B.Cu) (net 1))
 (segment (start 50.02316 91.28) (end 43.56 91.28) (width 0.25) (layer B.Cu) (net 1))
 (segment (start 51.46 91.28) (end 50.02316 91.28) (width 0.25) (layer B.Cu) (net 1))
 (segment (start 34.575999 90.264001) (end 33.56 91.28) (width 0.25) (layer B.Cu) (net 1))
 (segment (start 34.575999 75.295999) (end 34.575999 90.264001) (width 0.25) (layer B.Cu) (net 1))
 (segment (start 33.56 74.28) (end 34.575999 75.295999) (width 0.25) (layer B.Cu) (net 1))
 (segment (start 41.555839 94.721001) (end 37.001001 94.721001) (width 0.25) (layer B.Cu) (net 1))
 (segment (start 34.575999 92.295999) (end 33.56 91.28) (width 0.25) (layer B.Cu) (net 1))
 (segment (start 43.56 92.71684) (end 41.555839 94.721001) (width 0.25) (layer B.Cu) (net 1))
 (segment (start 37.001001 94.721001) (end 34.575999 92.295999) (width 0.25) (layer B.Cu) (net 1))
 (segment (start 43.56 91.28) (end 43.56 92.71684) (width 0.25) (layer B.Cu) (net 1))
 (segment (start 79.46 91.04) (end 79.46 91.28) (width 0.25) (layer F.Cu) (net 1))
 (segment (start 79.46 91.28) (end 79.58 91.28) (width 0.25) (layer F.Cu) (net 1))
 (segment (start 77.78 74.28) (end 75.02 74.28) (width 0.25) (layer B.Cu) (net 1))
 (segment (start 79.46 74.28) (end 77.78 74.28) (width 0.25) (layer B.Cu) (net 1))
 (segment (start 75.02 74.28) (end 72 77.3) (width 0.25) (layer B.Cu) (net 1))
 (segment (start 68.98 74.28) (end 61.46 74.28) (width 0.25) (layer B.Cu) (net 1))
 (segment (start 72 77.3) (end 68.98 74.28) (width 0.25) (layer B.Cu) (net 1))
 (segment (start 97.9 91.3) (end 98 91.4) (width 0.25) (layer B.Cu) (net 1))
 (segment (start 75.825001 61.474999) (end 75.499999 61.800001) (width 0.25) (layer B.Cu) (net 1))
 (segment (start 91.114999 61.474999) (end 75.825001 61.474999) (width 0.25) (layer B.Cu) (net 1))
 (segment (start 75.499999 61.800001) (end 74.5 62.8) (width 0.25) (layer B.Cu) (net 1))
 (segment (start 92.5 62.86) (end 91.114999 61.474999) (width 0.25) (layer B.Cu) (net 1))
 (segment (start 59.45 79.37) (end 56.46 76.38) (width 0.25) (layer B.Cu) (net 19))
 (segment (start 103.8986 80.132) (end 102.112 80.132) (width 0.25) (layer B.Cu) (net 19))
 (segment (start 102.112 80.132) (end 101.35 79.37) (width 0.25) (layer B.Cu) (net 19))
 (segment (start 101.35 79.37) (end 59.45 79.37) (width 0.25) (layer B.Cu) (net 19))
 (segment (start 103.448009 82.854999) (end 104.420361 82.854999) (width 0.25) (layer F.Cu) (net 2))
 (segment (start 103.564999 82.854999) (end 104.420361 82.854999) (width 0.25) (layer F.Cu) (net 2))
 (segment (start 100.3383 79.1117) (end 103.8986 82.672) (width 0.25) (layer F.Cu) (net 2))
 (segment (start 99.0683 79.1117) (end 100.3383 79.1117) (width 0.25) (layer F.Cu) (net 2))
 (segment (start 79.2 77.3) (end 81.3 79.4) (width 0.25) (layer F.Cu) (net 2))
 (segment (start 77 77.3) (end 79.2 77.3) (width 0.25) (layer F.Cu) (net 2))
 (segment (start 99.0683 79.1117) (end 81.3 79.4) (width 0.25) (layer F.Cu) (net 2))
 (segment (start 104.985601 84.124999) (end 104.660599 84.450001) (width 0.25) (layer F.Cu) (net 18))
 (segment (start 104.985601 82.150239) (end 104.985601 84.124999) (width 0.25) (layer F.Cu) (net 18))
 (segment (start 104.420361 81.584999) (end 104.985601 82.150239) (width 0.25) (layer F.Cu) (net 18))
 (segment (start 104.660599 84.450001) (end 103.8986 85.212) (width 0.25) (layer F.Cu) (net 18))
 (segment (start 103.564999 81.584999) (end 104.420361 81.584999) (width 0.25) (layer F.Cu) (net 18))
 (segment (start 99.34 77.36) (end 103.564999 81.584999) (width 0.25) (layer F.Cu) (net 18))
 (segment (start 94.92 77.36) (end 99.34 77.36) (width 0.25) (layer F.Cu) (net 18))
 (segment (start 103.136601 86.990001) (end 103.009999 86.990001) (width 0.25) (layer B.Cu) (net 17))
 (segment (start 103.8986 87.752) (end 103.136601 86.990001) (width 0.25) (layer B.Cu) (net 17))
 (segment (start 103.8986 87.752) (end 102 85.8534) (width 0.25) (layer B.Cu) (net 17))
 (segment (start 102 85.8534) (end 102 82.9) (width 0.25) (layer B.Cu) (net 17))
 (segment (start 99.6 80.5) (end 95 80.5) (width 0.25) (layer B.Cu) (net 17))
 (segment (start 102 82.9) (end 99.6 80.5) (width 0.25) (layer B.Cu) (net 17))
 (segment (start 90.475318 93.38) (end 74.46 93.38) (width 0.25) (layer F.Cu) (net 16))
 (segment (start 94.325317 89.530001) (end 90.475318 93.38) (width 0.25) (layer F.Cu) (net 16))
 (segment (start 103.136601 89.530001) (end 94.325317 89.530001) (width 0.25) (layer F.Cu) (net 16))
 (segment (start 103.8986 90.292) (end 103.136601 89.530001) (width 0.25) (layer F.Cu) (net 16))
 (segment (start 103.448009 92.649001) (end 104.420361 92.649001) (width 0.25) (layer F.Cu) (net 15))
 (segment (start 58.96 95.88) (end 56.46 93.38) (width 0.25) (layer F.Cu) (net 15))
 (segment (start 85.78 95.88) (end 88.6 98.7) (width 0.25) (layer F.Cu) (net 15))
 (segment (start 85.78 95.88) (end 58.96 95.88) (width 0.25) (layer F.Cu) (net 15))
 (segment (start 98.0306 98.7) (end 103.8986 92.832) (width 0.25) (layer F.Cu) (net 15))
 (segment (start 88.6 98.7) (end 98.0306 98.7) (width 0.25) (layer F.Cu) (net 15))
 (segment (start 107.871599 68.884999) (end 118.356601 79.370001) (width 0.25) (layer B.Cu) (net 4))
 (segment (start 103.484999 68.884999) (end 107.871599 68.884999) (width 0.25) (layer B.Cu) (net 4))
 (segment (start 118.356601 79.370001) (end 119.1186 80.132) (width 0.25) (layer B.Cu) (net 4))
 (segment (start 103.034999 68.434999) (end 103.484999 68.884999) (width 0.25) (layer B.Cu) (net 4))
 (segment (start 88.16 68.434999) (end 103.034999 68.434999) (width 0.25) (layer B.Cu) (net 4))
 (segment (start 82.525001 62.8) (end 88.16 68.434999) (width 0.25) (layer B.Cu) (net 4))
 (segment (start 77 62.8) (end 82.525001 62.8) (width 0.25) (layer B.Cu) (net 4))
 (segment (start 78.899999 72.285001) (end 72 65.385002) (width 0.25) (layer B.Cu) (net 3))
 (segment (start 99.360001 72.285001) (end 78.899999 72.285001) (width 0.25) (layer B.Cu) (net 3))
 (segment (start 100.220003 71.424999) (end 99.360001 72.285001) (width 0.25) (layer B.Cu) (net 3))
 (segment (start 107.871599 71.424999) (end 100.220003 71.424999) (width 0.25) (layer B.Cu) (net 3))
 (segment (start 72 64.214213) (end 72 62.8) (width 0.25) (layer B.Cu) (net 3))
 (segment (start 72 65.385002) (end 72 64.214213) (width 0.25) (layer B.Cu) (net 3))
 (segment (start 119.1186 82.672) (end 107.871599 71.424999) (width 0.25) (layer B.Cu) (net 3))
 (segment (start 118.356601 85.973999) (end 119.1186 85.212) (width 0.25) (layer F.Cu) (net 12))
 (segment (start 112.951599 91.379001) (end 118.356601 85.973999) (width 0.25) (layer F.Cu) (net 12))
 (segment (start 103.720999 91.379001) (end 112.951599 91.379001) (width 0.25) (layer F.Cu) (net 12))
 (segment (start 93.915999 94.415999) (end 100.784001 94.415999) (width 0.25) (layer F.Cu) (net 12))
 (segment (start 92.9 93.4) (end 93.915999 94.415999) (width 0.25) (layer F.Cu) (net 12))
 (segment (start 100.9 94.3) (end 103.720999 91.379001) (width 0.25) (layer F.Cu) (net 12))
 (segment (start 100.784001 94.415999) (end 100.9 94.3) (width 0.25) (layer F.Cu) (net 12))
 (segment (start 42.126009 89.813991) (end 100.227847 89.813991) (width 0.25) (layer B.Cu) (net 5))
 (segment (start 38.56 93.38) (end 42.126009 89.813991) (width 0.25) (layer B.Cu) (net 5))
 (segment (start 117.665601 89.204999) (end 118.356601 88.513999) (width 0.25) (layer B.Cu) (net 5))
 (segment (start 118.356601 88.513999) (end 119.1186 87.752) (width 0.25) (layer B.Cu) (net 5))
 (segment (start 100.836839 89.204999) (end 117.665601 89.204999) (width 0.25) (layer B.Cu) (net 5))
 (segment (start 100.227847 89.813991) (end 100.836839 89.204999) (width 0.25) (layer B.Cu) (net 5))
 (segment (start 103.136601 74.290001) (end 103.8986 75.052) (width 0.25) (layer F.Cu) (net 6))
 (segment (start 57.916319 72.938999) (end 101.785599 72.938999) (width 0.25) (layer F.Cu) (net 6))
 (segment (start 101.785599 72.938999) (end 103.136601 74.290001) (width 0.25) (layer F.Cu) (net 6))
 (segment (start 54.475318 76.38) (end 57.916319 72.938999) (width 0.25) (layer F.Cu) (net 6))
 (segment (start 38.56 76.38) (end 54.475318 76.38) (width 0.25) (layer F.Cu) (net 6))
 (segment (start 95 64.11) (end 95 62.86) (width 0.25) (layer B.Cu) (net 22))
 (segment (start 103.8986 64.892) (end 95.762 64.892) (width 0.25) (layer B.Cu) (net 22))
 (segment (start 95 64.13) (end 95 62.86) (width 0.25) (layer B.Cu) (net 22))
 (segment (start 95.762 64.892) (end 95 64.13) (width 0.25) (layer B.Cu) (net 22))
 (segment (start 94.572 67.432) (end 103.8986 67.432) (width 0.25) (layer B.Cu) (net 21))
 (segment (start 90 62.86) (end 94.572 67.432) (width 0.25) (layer B.Cu) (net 21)))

